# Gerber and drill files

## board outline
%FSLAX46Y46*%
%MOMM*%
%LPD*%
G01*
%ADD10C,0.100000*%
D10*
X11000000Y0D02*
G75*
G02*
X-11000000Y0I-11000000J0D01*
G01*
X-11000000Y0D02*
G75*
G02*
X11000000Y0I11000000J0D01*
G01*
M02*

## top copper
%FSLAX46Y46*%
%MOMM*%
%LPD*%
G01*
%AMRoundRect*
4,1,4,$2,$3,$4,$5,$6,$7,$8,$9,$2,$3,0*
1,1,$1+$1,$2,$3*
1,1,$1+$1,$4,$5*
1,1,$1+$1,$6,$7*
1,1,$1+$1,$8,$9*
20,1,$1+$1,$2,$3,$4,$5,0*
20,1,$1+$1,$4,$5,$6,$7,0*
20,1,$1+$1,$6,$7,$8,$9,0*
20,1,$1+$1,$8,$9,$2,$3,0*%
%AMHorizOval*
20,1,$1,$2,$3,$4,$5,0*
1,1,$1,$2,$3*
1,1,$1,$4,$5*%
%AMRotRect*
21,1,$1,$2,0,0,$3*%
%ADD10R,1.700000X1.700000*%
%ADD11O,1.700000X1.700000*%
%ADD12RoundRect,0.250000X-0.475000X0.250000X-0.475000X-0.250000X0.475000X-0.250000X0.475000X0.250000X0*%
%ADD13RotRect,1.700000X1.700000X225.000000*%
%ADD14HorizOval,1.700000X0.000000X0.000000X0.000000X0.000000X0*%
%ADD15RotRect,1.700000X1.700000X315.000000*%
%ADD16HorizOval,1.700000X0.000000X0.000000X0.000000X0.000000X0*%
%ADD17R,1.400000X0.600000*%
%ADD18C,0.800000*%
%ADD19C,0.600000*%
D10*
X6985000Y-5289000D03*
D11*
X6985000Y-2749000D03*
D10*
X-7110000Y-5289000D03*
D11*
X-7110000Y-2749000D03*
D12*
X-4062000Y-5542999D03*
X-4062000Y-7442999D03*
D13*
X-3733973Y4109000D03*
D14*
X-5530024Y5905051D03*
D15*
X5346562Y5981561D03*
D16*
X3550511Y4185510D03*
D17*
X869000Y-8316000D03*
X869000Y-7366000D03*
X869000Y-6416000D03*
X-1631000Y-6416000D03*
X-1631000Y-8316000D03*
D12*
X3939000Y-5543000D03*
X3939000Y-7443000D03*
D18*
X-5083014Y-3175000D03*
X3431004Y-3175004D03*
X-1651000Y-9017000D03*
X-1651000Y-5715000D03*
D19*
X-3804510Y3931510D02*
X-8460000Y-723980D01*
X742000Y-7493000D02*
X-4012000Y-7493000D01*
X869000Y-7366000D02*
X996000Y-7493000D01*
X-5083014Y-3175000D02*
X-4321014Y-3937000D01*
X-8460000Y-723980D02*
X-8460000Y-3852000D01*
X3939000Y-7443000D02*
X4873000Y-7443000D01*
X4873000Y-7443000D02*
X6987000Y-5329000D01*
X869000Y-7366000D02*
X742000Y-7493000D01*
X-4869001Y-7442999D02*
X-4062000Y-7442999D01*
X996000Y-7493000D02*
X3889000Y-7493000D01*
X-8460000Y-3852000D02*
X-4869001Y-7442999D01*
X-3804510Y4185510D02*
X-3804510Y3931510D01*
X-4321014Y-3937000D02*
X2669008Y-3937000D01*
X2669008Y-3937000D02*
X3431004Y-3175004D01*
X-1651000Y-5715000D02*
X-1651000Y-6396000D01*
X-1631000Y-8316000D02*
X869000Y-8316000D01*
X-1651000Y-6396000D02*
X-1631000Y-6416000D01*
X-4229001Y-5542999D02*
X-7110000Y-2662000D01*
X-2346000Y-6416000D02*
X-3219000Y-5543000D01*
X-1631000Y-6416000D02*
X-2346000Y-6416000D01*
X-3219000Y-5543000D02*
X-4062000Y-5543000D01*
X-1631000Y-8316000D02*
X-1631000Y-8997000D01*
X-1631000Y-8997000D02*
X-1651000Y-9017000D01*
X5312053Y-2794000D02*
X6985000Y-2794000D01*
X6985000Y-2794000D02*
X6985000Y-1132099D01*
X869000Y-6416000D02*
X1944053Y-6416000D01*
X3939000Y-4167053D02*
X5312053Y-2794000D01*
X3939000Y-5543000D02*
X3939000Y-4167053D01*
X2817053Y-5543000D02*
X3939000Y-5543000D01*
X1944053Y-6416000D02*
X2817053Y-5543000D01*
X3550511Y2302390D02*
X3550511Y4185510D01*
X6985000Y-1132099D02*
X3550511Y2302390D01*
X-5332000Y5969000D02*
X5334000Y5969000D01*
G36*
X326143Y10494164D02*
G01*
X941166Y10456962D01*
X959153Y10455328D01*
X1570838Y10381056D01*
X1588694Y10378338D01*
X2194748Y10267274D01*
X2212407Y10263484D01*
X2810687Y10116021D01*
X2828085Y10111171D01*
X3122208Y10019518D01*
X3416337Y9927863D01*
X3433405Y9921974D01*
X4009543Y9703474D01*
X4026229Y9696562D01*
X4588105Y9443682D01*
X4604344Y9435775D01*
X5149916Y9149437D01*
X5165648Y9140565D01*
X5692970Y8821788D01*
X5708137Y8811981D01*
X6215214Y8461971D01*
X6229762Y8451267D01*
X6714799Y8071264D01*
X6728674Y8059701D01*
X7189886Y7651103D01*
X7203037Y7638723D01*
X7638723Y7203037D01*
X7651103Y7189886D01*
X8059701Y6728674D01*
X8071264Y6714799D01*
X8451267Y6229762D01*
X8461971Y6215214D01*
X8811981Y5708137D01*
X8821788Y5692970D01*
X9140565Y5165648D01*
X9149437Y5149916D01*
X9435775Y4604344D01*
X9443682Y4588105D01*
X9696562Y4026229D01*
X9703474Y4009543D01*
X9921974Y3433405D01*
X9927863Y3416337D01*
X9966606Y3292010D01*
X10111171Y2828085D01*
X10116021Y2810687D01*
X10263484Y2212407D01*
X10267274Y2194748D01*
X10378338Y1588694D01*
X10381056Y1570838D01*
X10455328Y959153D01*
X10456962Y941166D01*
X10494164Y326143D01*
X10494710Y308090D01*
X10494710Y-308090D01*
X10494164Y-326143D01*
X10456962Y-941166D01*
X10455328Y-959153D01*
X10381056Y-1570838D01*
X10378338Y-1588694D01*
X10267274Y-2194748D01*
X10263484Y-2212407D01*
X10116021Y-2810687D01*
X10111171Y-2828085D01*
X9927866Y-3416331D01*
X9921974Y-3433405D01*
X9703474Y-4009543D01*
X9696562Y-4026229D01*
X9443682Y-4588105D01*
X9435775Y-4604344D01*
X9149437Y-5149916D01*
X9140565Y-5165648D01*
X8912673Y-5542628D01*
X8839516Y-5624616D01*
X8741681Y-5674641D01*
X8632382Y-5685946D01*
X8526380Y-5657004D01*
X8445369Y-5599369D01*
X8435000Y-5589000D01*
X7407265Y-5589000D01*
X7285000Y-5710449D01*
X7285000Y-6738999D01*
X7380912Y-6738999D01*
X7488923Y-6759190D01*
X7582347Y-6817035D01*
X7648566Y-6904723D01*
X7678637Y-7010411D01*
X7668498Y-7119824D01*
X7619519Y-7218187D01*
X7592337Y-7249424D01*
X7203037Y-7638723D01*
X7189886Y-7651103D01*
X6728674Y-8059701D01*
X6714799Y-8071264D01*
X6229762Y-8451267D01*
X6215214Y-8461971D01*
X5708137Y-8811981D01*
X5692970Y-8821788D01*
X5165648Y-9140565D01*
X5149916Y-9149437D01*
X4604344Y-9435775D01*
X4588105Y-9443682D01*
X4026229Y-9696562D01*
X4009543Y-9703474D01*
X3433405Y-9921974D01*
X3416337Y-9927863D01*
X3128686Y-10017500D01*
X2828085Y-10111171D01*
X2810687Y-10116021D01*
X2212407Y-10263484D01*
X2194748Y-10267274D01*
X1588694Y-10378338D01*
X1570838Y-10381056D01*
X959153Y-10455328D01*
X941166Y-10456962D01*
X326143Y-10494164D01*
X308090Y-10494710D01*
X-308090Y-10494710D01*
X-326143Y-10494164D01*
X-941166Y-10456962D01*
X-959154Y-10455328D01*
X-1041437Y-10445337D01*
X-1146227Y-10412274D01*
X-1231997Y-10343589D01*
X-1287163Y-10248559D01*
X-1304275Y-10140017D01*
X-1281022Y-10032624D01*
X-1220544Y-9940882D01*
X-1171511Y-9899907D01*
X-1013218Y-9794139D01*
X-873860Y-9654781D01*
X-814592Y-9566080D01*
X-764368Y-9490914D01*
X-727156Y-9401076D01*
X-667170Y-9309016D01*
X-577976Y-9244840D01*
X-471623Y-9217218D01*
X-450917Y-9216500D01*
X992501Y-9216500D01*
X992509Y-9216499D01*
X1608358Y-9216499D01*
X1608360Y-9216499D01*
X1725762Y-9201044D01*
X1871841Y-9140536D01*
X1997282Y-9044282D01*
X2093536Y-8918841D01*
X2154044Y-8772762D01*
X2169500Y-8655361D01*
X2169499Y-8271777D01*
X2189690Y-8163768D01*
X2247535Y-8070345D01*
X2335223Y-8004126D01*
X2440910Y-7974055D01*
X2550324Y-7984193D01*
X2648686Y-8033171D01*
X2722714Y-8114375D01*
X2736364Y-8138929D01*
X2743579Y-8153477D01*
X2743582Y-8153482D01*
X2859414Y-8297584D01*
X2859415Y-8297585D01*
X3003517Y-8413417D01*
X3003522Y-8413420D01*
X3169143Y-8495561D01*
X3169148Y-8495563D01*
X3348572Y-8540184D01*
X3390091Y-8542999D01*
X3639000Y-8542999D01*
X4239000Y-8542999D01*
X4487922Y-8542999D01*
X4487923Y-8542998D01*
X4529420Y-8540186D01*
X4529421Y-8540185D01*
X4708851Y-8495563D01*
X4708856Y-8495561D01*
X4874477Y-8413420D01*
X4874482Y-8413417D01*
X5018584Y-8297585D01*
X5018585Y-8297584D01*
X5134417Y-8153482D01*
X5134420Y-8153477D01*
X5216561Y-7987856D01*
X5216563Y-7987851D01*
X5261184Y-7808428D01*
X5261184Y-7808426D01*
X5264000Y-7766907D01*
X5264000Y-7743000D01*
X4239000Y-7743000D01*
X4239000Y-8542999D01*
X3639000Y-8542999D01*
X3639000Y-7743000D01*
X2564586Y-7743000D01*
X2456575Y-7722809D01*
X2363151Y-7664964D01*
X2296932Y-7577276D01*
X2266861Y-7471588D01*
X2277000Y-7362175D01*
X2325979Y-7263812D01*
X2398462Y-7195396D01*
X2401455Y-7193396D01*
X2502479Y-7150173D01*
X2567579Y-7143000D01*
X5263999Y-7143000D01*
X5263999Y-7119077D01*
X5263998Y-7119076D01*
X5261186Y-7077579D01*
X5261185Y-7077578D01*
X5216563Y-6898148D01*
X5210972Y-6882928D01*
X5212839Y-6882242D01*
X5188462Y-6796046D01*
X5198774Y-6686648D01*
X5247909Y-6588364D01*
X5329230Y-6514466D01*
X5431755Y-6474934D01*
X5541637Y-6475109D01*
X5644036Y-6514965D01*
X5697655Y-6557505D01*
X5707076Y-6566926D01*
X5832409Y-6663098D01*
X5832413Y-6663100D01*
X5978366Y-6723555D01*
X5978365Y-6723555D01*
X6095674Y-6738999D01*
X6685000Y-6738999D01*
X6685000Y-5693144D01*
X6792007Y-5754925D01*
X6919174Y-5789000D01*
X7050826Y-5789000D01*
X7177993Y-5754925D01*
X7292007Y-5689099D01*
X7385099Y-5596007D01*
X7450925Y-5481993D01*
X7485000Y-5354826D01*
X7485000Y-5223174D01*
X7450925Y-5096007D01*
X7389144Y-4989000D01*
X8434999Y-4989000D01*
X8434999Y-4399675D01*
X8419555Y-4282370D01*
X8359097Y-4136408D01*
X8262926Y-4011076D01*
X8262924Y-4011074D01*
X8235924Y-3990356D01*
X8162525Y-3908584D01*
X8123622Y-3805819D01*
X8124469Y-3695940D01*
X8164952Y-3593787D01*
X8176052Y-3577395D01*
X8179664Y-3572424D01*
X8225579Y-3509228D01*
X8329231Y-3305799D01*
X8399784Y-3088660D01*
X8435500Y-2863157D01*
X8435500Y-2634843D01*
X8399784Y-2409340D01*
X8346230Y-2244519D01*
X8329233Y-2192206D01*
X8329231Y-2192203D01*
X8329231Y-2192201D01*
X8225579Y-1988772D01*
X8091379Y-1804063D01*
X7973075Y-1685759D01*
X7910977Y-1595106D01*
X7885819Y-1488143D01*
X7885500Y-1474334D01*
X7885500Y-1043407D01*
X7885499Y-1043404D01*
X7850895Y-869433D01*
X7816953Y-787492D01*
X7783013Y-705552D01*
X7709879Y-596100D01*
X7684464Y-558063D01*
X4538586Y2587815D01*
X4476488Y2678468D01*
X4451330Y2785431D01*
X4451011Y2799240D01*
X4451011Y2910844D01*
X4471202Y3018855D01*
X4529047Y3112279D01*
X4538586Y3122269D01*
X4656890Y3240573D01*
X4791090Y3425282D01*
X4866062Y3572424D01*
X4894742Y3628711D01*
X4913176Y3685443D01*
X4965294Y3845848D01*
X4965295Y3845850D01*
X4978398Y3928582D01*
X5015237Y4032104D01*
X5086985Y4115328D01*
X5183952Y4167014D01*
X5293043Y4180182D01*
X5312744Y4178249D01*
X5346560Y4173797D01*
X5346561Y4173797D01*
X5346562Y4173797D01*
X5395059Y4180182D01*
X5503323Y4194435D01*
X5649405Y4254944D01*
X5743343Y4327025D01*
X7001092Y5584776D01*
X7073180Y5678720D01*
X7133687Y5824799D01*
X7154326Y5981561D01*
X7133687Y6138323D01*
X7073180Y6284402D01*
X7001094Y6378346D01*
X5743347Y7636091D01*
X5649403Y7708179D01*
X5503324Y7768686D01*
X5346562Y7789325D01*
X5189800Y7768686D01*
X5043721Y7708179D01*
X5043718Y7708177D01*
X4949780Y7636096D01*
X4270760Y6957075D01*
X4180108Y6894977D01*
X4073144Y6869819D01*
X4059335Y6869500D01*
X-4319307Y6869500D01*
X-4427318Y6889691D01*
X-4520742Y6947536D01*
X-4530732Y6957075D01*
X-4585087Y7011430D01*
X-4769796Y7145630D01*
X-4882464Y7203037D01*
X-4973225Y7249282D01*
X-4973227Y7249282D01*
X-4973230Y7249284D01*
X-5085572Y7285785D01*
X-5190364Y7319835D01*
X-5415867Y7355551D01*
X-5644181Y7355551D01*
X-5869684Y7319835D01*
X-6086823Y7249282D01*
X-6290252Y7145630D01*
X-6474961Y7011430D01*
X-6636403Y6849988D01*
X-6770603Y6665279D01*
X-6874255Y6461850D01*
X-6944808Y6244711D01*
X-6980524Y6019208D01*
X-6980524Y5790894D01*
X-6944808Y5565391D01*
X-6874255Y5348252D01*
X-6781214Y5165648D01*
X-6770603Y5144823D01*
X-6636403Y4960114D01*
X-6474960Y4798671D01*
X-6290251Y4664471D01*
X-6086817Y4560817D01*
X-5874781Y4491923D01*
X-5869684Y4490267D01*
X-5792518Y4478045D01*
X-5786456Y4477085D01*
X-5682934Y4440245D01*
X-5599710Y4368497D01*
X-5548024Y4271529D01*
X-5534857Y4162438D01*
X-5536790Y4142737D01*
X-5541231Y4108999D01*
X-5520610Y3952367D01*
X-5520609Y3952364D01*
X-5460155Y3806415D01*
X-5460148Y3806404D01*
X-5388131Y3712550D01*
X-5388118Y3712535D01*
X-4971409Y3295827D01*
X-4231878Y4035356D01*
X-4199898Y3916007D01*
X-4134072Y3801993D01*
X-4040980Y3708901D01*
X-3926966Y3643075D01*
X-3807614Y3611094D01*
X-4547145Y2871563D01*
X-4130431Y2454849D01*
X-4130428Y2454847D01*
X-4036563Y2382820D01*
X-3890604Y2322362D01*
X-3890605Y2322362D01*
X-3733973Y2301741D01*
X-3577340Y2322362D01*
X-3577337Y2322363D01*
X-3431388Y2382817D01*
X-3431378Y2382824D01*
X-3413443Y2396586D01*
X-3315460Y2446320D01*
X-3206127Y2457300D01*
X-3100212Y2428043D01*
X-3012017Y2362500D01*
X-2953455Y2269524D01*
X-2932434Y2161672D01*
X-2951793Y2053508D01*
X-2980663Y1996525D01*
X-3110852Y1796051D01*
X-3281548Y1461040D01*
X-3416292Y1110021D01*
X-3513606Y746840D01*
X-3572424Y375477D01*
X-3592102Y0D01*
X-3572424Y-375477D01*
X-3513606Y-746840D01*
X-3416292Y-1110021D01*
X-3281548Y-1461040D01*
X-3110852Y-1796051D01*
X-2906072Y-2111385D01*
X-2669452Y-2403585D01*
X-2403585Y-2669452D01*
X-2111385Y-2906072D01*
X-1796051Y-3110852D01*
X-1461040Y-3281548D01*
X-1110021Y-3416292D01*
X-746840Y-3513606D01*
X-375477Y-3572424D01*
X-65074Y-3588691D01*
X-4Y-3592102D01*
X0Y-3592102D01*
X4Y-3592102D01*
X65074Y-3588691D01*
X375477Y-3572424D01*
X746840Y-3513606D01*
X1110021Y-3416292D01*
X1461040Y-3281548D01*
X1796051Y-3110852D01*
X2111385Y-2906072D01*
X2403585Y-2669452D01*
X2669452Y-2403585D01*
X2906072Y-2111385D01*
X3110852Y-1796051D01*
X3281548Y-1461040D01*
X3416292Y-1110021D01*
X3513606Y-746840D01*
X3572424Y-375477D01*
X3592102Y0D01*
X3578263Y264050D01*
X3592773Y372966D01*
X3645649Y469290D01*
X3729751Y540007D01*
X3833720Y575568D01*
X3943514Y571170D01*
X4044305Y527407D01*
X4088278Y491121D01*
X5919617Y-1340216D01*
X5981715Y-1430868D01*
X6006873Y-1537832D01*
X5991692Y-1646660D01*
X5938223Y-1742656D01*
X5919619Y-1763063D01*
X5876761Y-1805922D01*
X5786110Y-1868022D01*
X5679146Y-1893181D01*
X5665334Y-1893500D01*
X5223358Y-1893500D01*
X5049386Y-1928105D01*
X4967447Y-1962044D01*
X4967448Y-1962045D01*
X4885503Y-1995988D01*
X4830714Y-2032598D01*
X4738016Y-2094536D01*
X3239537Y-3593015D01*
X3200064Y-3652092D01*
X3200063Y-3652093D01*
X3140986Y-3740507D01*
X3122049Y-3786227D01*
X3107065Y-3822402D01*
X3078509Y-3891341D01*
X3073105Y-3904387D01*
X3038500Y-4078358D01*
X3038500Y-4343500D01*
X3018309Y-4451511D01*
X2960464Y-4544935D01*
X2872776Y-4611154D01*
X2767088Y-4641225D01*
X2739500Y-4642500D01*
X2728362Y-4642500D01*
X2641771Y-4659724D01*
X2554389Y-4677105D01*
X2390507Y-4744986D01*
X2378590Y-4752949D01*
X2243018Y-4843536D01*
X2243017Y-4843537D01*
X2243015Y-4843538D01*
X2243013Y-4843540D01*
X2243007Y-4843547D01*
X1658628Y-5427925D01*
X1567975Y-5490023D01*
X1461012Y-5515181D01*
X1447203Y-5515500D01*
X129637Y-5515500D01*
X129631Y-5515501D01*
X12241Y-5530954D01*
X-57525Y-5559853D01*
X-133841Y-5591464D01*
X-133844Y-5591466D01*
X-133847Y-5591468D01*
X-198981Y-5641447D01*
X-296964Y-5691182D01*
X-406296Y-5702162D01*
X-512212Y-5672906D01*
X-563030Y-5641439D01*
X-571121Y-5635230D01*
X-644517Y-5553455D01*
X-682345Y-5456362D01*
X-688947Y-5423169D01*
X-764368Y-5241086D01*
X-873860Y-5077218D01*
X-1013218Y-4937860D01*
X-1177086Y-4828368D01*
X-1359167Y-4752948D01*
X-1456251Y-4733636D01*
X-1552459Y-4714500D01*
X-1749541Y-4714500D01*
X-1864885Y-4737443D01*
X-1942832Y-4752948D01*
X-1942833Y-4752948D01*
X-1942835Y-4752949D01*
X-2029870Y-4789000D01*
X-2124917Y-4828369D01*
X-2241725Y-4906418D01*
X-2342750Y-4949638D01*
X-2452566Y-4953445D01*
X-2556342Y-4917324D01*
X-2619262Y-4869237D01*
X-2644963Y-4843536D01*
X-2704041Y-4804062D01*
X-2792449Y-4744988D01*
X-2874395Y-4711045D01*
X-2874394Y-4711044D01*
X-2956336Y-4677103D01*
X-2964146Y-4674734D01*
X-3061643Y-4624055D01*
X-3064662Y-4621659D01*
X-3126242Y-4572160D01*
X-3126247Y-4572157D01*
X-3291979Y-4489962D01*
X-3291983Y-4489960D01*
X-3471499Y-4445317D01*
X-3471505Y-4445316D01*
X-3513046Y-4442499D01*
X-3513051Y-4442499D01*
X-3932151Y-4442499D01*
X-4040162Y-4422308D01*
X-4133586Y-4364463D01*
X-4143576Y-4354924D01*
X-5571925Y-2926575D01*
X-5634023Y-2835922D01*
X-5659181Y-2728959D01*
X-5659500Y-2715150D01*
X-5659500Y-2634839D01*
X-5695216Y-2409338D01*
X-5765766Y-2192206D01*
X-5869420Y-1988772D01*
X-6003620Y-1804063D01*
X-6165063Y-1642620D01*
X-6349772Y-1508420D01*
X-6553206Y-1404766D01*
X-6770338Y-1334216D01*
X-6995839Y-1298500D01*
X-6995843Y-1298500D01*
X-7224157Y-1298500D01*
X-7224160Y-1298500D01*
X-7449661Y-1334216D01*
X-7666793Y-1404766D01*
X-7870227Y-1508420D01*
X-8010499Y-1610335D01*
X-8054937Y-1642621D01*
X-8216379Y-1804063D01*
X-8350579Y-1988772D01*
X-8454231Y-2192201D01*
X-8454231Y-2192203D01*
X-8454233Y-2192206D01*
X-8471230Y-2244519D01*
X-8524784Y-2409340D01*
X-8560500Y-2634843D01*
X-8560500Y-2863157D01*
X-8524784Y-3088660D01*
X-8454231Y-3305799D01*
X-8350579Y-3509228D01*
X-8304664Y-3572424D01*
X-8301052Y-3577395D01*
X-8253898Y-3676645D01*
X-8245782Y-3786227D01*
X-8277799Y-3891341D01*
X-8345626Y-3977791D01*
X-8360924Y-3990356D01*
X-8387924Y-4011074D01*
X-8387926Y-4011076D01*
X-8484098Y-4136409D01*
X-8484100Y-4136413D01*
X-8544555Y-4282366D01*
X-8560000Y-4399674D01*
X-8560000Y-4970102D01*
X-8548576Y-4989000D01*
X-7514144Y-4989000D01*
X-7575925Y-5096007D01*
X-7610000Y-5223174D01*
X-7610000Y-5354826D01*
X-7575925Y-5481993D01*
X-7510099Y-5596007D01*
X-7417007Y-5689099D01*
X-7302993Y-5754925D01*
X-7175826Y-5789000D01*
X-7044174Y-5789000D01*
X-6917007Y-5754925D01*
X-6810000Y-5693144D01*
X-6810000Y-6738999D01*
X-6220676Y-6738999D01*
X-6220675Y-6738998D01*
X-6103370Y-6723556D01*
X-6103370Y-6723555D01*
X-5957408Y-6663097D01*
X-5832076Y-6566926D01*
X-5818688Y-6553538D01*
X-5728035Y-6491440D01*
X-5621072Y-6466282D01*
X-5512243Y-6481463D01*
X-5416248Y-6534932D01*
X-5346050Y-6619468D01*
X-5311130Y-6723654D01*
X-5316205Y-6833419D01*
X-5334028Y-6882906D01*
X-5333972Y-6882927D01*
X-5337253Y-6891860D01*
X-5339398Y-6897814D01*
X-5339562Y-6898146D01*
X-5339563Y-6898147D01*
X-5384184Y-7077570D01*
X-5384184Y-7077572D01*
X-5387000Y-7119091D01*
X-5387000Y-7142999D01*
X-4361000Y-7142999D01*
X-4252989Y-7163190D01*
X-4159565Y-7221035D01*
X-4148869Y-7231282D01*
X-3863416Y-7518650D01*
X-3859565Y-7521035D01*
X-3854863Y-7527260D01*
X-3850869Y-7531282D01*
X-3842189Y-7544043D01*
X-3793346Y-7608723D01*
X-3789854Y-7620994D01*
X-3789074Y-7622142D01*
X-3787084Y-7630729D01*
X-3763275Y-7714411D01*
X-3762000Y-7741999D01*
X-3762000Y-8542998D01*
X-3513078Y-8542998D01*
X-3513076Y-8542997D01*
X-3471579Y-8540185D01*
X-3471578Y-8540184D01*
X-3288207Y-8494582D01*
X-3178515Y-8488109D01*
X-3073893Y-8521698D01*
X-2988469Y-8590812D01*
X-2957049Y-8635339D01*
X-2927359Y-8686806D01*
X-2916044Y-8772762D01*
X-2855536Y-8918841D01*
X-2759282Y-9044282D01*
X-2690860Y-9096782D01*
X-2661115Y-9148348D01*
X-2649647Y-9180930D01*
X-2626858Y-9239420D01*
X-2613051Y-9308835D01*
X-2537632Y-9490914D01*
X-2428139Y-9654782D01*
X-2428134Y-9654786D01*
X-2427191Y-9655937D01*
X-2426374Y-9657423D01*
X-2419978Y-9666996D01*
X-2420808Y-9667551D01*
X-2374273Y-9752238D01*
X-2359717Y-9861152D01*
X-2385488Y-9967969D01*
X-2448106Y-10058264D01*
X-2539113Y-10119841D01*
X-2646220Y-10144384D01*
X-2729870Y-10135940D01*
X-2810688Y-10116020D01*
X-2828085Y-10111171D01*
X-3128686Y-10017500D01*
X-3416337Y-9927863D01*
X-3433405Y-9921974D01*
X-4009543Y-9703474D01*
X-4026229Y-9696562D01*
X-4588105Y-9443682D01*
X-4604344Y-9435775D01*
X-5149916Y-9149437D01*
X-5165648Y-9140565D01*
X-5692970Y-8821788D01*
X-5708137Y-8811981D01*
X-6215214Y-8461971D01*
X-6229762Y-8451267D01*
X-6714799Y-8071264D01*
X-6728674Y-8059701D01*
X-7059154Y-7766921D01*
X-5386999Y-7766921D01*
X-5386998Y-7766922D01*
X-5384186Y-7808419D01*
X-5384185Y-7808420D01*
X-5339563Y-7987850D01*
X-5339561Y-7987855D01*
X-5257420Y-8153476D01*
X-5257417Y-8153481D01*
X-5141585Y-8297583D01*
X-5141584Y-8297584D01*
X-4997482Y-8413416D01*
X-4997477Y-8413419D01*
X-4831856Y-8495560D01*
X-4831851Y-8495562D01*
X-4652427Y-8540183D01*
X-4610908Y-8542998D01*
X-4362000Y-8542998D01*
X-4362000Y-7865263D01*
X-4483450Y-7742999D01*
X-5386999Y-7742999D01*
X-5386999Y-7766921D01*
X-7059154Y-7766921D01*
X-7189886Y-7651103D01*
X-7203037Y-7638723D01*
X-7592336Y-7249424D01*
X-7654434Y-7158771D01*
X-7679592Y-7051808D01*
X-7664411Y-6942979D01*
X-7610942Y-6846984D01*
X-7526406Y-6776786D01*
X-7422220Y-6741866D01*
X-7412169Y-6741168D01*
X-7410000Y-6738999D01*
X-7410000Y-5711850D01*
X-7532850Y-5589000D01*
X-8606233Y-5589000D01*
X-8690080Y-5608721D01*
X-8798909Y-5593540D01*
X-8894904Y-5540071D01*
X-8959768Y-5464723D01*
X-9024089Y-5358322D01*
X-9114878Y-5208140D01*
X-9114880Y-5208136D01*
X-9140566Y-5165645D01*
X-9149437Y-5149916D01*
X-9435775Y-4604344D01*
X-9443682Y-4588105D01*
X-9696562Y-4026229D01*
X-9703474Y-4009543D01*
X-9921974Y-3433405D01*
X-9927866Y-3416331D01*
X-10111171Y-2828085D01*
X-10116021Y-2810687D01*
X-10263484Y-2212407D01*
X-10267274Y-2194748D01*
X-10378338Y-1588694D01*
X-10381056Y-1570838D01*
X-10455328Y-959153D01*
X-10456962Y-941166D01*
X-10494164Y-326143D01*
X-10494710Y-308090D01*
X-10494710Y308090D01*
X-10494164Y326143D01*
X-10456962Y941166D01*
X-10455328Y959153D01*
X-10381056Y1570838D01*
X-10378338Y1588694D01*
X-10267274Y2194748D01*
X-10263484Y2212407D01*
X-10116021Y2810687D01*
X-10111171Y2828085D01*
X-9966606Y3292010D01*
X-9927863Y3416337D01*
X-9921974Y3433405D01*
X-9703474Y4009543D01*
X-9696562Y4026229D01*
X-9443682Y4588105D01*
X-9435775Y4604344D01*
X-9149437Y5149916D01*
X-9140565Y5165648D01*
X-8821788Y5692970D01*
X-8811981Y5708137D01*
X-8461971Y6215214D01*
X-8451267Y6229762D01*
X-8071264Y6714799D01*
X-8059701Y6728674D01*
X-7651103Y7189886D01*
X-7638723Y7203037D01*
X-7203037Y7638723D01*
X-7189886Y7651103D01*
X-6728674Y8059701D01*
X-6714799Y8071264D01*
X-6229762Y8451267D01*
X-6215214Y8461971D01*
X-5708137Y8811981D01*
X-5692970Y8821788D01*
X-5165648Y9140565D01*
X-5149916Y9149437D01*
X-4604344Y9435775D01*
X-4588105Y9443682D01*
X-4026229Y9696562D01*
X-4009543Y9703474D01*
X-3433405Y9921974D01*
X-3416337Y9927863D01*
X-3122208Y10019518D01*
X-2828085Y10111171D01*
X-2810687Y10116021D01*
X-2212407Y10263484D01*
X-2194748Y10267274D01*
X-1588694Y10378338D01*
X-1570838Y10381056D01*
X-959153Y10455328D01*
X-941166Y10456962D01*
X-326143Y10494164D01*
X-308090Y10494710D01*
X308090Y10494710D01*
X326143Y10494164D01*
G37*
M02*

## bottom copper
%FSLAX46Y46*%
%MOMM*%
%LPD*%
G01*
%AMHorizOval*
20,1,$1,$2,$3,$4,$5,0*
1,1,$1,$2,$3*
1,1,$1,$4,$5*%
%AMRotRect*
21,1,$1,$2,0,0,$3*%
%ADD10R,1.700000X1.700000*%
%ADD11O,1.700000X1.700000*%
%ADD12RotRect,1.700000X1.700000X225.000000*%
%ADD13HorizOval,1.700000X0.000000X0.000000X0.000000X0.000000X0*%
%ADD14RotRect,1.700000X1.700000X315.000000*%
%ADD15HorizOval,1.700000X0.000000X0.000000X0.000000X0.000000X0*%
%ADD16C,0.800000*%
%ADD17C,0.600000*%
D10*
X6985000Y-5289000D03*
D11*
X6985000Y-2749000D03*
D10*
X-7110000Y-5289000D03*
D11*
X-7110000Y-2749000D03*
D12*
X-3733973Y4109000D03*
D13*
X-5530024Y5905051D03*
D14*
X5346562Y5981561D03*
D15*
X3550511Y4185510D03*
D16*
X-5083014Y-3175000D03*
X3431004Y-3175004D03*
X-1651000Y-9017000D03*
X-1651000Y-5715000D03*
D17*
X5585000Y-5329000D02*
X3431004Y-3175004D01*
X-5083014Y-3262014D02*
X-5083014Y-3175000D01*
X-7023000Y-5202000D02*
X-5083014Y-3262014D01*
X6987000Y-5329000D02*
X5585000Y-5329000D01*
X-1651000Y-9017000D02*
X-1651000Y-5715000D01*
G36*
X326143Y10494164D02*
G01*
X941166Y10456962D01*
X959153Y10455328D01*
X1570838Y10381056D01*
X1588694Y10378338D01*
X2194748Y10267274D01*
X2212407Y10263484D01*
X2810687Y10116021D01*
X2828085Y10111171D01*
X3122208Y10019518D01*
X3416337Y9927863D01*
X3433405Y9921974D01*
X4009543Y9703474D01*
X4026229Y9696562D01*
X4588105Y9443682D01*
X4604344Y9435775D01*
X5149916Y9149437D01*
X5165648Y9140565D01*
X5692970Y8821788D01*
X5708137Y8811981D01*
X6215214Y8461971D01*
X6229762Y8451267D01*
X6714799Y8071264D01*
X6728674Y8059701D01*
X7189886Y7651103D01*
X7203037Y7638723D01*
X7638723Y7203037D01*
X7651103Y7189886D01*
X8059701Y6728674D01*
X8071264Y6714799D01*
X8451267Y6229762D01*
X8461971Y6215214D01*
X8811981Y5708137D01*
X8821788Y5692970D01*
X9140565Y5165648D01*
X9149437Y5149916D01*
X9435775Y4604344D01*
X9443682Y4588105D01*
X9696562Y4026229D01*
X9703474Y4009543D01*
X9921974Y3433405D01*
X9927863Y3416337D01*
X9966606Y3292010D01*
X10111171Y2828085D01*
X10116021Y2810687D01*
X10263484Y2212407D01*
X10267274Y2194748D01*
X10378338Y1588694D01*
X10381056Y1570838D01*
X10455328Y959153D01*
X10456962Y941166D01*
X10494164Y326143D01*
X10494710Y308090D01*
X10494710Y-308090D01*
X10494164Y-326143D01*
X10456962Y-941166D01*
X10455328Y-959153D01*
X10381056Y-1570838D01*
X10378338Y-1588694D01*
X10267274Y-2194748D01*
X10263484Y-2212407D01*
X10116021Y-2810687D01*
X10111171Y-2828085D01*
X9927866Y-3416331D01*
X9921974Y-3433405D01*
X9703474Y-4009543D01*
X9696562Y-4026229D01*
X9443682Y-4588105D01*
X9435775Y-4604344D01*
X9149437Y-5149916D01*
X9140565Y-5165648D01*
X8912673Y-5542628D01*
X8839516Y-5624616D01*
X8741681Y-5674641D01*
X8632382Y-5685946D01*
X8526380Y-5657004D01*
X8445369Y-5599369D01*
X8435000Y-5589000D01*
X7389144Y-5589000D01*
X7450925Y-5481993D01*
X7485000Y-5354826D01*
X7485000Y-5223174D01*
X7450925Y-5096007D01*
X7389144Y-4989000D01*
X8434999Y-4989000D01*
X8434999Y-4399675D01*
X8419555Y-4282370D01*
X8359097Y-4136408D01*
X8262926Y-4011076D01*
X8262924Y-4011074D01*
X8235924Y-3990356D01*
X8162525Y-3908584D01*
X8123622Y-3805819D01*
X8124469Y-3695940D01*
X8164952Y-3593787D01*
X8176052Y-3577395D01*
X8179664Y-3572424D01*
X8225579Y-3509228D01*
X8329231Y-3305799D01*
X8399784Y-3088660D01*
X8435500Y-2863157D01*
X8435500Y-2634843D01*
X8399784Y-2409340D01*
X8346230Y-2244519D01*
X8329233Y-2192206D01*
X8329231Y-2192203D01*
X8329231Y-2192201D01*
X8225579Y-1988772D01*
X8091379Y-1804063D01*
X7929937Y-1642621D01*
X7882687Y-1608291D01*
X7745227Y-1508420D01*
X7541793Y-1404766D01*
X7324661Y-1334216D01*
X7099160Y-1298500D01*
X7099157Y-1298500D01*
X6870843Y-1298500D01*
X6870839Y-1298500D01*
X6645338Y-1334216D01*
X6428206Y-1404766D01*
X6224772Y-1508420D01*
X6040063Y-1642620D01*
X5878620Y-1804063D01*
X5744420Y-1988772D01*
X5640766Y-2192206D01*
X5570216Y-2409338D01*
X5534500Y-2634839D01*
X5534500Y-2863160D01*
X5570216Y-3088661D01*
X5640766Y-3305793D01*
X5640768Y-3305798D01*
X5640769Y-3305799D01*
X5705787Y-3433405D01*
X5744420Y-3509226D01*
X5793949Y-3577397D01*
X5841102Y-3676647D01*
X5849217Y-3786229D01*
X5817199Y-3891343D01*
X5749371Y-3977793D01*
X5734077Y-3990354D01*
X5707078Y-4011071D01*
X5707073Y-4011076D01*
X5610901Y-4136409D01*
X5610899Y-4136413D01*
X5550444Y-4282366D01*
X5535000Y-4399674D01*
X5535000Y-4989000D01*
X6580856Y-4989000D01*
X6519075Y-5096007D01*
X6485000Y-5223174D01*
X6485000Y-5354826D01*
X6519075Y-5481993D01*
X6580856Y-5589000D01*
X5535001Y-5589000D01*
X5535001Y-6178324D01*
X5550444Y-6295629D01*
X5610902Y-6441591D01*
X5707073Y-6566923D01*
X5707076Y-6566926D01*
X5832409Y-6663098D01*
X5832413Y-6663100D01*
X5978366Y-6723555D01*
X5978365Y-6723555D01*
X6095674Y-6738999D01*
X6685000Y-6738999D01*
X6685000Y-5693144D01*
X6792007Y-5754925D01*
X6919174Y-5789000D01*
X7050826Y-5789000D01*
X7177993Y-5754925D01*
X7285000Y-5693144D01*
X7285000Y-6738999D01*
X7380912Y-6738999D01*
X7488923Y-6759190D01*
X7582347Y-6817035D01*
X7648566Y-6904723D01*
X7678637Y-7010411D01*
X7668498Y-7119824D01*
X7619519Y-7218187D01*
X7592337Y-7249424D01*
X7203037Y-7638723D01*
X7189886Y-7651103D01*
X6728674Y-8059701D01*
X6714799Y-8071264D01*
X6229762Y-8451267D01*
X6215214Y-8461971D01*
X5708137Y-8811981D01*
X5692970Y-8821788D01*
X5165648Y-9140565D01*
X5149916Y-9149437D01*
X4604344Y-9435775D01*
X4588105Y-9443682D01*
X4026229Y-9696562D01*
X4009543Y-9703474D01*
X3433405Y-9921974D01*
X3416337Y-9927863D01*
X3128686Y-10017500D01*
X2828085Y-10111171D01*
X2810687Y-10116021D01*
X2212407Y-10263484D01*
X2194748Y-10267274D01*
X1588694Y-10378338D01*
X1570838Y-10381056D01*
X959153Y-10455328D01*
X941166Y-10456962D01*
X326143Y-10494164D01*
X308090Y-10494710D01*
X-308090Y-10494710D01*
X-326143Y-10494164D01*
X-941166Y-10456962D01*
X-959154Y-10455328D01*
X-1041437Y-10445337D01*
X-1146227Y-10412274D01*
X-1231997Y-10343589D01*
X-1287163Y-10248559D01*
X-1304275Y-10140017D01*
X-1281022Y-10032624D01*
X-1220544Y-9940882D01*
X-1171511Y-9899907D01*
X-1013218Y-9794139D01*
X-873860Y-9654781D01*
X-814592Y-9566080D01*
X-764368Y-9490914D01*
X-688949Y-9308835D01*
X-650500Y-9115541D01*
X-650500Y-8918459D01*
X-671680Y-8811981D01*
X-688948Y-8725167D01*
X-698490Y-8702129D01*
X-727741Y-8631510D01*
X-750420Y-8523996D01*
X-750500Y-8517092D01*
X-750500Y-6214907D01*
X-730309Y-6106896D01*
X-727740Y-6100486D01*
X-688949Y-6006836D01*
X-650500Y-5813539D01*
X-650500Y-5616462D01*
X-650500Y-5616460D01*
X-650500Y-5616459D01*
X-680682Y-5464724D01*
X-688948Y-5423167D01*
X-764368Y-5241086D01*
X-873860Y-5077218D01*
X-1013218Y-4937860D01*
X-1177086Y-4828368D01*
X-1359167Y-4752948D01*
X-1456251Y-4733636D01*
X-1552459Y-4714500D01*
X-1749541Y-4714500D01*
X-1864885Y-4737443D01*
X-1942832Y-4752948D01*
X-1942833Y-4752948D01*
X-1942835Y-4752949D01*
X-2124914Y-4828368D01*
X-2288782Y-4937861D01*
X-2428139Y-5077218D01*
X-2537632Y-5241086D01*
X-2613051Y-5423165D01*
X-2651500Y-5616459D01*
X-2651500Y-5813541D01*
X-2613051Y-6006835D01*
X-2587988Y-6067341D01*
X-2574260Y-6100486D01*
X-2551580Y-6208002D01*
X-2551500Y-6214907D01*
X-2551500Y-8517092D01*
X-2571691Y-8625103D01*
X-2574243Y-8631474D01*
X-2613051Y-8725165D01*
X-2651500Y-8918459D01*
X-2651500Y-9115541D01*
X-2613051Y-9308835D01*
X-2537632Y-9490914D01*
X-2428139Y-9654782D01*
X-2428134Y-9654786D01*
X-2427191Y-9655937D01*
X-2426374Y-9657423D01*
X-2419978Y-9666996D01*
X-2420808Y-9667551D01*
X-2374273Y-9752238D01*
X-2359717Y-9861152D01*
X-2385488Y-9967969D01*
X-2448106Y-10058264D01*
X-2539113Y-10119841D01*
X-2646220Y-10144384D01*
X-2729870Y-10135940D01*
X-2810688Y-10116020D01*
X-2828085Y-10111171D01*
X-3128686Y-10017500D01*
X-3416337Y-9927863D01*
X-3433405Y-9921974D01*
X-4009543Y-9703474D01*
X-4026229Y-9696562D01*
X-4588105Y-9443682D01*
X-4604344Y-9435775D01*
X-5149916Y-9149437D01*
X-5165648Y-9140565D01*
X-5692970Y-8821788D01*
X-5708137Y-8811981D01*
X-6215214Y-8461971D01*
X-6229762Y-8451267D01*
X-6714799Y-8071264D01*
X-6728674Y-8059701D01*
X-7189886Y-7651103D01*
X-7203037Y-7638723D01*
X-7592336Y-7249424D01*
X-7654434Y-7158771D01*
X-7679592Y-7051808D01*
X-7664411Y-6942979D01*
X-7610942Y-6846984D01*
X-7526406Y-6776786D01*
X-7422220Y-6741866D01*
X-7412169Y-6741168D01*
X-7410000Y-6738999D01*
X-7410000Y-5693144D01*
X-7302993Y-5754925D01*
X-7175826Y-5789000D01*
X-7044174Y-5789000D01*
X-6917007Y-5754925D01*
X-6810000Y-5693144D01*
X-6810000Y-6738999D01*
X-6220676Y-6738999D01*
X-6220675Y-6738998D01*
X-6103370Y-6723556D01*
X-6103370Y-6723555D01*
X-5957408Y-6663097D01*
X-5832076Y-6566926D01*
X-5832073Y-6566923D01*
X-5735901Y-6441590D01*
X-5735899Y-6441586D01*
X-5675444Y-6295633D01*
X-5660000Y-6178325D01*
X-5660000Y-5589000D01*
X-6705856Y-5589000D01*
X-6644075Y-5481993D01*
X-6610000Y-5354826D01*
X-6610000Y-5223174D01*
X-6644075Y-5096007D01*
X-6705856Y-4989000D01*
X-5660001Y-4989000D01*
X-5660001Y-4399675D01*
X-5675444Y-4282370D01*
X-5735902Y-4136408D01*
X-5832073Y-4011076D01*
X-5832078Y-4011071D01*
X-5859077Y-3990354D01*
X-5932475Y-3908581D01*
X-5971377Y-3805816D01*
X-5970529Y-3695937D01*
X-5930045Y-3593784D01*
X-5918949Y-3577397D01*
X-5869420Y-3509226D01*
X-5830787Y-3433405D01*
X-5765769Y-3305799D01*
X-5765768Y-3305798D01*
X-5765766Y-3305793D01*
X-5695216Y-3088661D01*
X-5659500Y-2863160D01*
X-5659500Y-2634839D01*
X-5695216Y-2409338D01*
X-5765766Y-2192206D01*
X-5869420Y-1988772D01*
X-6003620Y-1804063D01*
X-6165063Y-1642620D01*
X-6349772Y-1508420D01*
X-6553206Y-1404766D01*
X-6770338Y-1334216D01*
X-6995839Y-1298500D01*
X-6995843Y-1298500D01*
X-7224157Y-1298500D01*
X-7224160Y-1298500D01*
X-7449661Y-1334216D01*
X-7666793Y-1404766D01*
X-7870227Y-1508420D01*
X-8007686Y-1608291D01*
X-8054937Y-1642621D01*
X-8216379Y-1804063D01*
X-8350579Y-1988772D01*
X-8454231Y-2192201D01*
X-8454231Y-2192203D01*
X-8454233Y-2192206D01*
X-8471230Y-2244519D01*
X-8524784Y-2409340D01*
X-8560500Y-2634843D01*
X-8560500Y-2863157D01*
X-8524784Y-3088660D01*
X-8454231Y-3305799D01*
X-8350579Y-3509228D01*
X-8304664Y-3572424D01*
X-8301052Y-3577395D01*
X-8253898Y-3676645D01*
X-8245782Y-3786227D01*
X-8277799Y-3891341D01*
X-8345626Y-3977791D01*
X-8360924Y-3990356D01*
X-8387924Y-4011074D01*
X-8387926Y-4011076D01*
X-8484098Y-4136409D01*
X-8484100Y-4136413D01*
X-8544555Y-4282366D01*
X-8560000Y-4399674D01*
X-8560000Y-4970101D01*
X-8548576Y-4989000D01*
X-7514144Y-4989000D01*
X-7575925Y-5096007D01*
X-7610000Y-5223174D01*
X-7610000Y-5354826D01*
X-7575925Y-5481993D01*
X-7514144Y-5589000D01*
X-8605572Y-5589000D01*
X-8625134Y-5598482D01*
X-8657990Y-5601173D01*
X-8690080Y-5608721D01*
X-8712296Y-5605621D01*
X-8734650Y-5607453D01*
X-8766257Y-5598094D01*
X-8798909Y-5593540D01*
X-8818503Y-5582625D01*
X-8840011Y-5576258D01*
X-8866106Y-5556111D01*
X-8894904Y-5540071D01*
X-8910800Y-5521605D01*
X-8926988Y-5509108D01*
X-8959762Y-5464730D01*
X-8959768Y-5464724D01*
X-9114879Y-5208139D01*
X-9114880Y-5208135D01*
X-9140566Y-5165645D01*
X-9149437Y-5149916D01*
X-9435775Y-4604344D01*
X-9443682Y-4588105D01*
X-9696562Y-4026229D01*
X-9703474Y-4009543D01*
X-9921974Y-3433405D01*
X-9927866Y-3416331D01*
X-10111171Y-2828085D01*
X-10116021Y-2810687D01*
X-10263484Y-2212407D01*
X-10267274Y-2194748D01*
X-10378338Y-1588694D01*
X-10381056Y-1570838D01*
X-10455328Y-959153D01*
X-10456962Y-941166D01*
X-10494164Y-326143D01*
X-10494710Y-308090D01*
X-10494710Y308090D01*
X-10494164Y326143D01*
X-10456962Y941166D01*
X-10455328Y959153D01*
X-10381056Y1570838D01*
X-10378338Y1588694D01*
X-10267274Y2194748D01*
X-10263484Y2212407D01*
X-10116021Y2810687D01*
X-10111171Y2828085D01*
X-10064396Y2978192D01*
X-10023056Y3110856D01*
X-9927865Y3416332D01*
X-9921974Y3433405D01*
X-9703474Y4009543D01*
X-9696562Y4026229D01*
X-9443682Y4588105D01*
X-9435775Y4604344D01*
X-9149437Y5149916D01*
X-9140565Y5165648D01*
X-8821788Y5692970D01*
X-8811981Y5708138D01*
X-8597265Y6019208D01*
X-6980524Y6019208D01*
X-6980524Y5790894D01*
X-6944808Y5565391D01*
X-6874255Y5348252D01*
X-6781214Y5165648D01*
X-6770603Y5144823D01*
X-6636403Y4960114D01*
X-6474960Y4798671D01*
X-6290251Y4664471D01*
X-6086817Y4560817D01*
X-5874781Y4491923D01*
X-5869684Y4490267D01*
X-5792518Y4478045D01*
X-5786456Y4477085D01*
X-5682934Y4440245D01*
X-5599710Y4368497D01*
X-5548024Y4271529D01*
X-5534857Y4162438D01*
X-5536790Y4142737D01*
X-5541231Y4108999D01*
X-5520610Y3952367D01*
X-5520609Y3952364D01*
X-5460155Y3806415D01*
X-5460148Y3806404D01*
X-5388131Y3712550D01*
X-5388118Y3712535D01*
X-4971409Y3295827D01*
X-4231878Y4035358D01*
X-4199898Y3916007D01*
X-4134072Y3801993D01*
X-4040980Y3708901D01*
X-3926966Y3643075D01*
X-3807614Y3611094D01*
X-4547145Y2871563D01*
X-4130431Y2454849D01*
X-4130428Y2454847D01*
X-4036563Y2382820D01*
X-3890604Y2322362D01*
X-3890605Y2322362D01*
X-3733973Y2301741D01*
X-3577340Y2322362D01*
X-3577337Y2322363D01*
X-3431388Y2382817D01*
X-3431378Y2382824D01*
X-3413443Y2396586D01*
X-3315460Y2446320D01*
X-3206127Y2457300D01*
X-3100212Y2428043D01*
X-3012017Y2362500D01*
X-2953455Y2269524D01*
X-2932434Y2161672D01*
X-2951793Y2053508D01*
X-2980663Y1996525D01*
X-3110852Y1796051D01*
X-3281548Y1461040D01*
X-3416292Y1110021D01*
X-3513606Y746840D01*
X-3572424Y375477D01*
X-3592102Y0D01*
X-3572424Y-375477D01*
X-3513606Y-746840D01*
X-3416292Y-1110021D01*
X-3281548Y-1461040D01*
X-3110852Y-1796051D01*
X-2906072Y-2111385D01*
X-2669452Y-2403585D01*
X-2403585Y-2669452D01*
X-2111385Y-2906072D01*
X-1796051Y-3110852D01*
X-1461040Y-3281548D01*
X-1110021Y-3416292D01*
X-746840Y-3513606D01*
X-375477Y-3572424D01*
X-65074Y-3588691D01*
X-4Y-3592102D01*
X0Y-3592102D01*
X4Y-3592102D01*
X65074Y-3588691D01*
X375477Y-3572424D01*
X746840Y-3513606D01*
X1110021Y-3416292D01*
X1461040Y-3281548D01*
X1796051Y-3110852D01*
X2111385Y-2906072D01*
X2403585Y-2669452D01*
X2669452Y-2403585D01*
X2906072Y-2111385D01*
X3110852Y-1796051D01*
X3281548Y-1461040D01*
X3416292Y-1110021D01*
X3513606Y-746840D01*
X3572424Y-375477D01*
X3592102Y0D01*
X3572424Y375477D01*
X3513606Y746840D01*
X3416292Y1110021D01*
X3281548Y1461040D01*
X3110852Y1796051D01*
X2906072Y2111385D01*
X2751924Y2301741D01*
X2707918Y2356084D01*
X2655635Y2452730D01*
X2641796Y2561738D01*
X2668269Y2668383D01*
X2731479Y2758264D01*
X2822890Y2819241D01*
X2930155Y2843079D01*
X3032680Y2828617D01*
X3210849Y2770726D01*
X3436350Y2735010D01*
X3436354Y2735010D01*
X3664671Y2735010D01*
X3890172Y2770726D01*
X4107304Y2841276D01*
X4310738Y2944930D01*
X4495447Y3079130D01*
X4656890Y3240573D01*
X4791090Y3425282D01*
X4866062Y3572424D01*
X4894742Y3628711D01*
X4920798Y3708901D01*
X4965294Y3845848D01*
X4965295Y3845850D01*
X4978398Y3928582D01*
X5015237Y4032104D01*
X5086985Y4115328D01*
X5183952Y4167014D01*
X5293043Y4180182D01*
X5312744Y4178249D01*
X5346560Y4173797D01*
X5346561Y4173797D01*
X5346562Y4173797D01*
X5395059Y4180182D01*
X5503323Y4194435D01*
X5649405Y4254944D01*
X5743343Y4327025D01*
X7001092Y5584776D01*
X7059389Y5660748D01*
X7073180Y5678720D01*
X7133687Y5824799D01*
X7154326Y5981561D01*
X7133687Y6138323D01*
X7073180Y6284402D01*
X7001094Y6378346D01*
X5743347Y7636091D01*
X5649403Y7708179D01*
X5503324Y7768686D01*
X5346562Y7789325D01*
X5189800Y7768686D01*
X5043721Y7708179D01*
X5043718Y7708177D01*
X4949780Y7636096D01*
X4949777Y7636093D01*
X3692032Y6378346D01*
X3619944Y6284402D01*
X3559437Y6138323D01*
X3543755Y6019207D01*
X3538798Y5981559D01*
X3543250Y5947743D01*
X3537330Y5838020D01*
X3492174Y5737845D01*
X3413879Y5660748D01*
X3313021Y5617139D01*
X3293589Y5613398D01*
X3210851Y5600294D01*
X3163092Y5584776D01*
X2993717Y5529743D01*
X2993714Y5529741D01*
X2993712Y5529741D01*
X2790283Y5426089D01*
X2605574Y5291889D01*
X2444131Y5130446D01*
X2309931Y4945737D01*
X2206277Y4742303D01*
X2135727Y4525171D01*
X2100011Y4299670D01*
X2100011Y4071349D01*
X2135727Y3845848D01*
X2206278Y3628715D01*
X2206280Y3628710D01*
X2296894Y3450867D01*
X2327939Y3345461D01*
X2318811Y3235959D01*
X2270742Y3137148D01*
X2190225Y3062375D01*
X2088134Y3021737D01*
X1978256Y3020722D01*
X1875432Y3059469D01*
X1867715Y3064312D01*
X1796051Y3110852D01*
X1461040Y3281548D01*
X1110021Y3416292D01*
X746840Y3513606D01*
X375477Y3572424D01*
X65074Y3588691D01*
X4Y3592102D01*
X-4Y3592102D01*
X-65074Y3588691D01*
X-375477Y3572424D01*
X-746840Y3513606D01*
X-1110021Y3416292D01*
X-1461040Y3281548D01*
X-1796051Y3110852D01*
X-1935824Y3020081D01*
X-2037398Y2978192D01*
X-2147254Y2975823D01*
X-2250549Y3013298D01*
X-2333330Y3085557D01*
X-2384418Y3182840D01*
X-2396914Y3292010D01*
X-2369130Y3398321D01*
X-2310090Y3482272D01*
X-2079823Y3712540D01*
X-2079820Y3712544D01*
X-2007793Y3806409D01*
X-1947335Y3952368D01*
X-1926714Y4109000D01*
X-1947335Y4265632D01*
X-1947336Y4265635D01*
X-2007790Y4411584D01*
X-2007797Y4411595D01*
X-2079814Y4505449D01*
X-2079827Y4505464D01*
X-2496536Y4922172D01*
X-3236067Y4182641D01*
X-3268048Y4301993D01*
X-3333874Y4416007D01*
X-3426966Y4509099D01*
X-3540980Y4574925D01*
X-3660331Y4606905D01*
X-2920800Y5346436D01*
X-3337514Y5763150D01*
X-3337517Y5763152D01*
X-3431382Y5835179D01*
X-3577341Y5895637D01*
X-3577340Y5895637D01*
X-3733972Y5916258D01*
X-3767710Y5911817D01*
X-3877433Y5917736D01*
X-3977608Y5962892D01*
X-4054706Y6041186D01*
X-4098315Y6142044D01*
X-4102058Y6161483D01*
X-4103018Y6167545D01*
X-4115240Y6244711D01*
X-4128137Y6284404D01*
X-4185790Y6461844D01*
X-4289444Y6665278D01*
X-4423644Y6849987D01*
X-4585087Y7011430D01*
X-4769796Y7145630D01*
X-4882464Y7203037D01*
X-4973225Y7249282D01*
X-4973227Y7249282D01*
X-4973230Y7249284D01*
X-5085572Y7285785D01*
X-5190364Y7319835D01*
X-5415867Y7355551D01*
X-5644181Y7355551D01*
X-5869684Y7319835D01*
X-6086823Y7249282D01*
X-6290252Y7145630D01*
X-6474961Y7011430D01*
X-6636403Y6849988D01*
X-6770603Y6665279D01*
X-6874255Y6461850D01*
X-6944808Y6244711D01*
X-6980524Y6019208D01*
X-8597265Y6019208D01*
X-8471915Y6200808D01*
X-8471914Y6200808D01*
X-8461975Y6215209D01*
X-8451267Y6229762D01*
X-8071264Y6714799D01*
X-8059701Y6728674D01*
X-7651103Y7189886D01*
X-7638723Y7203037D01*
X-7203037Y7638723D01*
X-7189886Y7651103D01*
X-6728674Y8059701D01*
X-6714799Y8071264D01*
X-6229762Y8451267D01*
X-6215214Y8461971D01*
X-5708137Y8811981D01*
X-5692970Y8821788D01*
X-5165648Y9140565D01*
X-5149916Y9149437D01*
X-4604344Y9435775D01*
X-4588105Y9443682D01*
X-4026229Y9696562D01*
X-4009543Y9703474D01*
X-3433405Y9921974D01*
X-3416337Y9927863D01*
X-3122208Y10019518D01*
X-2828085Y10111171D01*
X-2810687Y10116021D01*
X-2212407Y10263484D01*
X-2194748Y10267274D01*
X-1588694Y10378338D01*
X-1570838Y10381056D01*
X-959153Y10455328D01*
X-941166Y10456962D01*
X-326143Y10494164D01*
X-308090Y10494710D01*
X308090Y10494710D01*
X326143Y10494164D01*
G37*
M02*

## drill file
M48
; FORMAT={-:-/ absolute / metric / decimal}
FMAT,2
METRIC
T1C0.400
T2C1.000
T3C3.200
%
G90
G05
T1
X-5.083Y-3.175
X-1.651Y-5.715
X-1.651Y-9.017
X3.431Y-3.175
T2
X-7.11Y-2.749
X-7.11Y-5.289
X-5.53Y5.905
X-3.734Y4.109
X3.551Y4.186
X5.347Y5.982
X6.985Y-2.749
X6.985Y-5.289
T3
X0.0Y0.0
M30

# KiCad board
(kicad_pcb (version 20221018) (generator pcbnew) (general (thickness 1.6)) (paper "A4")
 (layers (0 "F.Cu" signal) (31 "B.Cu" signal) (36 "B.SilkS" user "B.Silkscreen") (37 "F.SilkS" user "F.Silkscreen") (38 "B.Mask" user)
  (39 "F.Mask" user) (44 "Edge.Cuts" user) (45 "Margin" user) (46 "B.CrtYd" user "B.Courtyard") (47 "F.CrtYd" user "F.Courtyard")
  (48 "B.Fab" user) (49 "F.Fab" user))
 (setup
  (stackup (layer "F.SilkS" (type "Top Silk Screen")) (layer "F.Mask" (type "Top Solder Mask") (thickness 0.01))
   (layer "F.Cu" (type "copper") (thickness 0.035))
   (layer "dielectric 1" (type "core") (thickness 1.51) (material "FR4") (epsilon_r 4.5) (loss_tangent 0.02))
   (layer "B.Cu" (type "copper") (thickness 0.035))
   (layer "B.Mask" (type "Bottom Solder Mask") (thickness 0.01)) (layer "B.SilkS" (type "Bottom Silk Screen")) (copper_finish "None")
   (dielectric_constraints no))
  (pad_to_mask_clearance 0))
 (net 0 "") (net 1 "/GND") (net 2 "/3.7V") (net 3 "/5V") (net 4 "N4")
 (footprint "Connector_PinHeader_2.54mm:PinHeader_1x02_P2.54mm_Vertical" (layer "F.Cu") (at 6.985 5.289 180)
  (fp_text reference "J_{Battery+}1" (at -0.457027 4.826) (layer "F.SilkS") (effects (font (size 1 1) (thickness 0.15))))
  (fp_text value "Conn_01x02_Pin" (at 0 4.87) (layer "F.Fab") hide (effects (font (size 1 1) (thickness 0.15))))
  (pad "1" thru_hole rect (at 0 0 180) (size 1.7 1.7) (drill 1) (layers "*.Cu" "*.Mask") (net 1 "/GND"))
  (pad "2" thru_hole oval (at 0 2.54 180) (size 1.7 1.7) (drill 1) (layers "*.Cu" "*.Mask") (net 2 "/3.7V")))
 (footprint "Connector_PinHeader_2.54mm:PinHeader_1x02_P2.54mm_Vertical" (layer "F.Cu") (at -7.11 5.289 180)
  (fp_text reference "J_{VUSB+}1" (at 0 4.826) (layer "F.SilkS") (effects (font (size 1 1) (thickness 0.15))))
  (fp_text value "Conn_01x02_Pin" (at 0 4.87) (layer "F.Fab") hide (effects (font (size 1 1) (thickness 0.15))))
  (pad "1" thru_hole rect (at 0 0 180) (size 1.7 1.7) (drill 1) (layers "*.Cu" "*.Mask") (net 1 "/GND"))
  (pad "2" thru_hole oval (at 0 2.54 180) (size 1.7 1.7) (drill 1) (layers "*.Cu" "*.Mask") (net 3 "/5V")))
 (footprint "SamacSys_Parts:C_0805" (layer "F.Cu") (at -4.062 6.476999 180)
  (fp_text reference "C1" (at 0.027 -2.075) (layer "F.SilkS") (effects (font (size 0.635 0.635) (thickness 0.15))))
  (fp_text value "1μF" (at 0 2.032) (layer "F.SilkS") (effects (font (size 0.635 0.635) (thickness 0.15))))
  (pad "1" smd roundrect (at 0 0.934 270) (size 1 1.45) (layers "F.Cu" "F.Paste" "F.Mask") (roundrect_rratio 0.25) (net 3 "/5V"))
  (pad "2" smd roundrect (at 0 -0.966 270) (size 1 1.45) (layers "F.Cu" "F.Paste" "F.Mask") (roundrect_rratio 0.25) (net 1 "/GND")))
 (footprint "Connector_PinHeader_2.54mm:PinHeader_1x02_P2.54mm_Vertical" (layer "F.Cu") (at -3.733973 -4.109 -135)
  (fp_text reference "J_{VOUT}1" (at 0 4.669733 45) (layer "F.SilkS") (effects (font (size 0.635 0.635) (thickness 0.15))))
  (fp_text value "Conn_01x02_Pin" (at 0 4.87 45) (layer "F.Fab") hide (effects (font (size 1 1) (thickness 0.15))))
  (pad "1" thru_hole rect (at 0 0 225) (size 1.7 1.7) (drill 1) (layers "*.Cu" "*.Mask") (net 1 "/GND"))
  (pad "2" thru_hole oval (at 0 2.54 225) (size 1.7 1.7) (drill 1) (layers "*.Cu" "*.Mask") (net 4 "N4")))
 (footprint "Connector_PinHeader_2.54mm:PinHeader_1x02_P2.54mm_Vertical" (layer "F.Cu") (at 5.346562 -5.981561 -45)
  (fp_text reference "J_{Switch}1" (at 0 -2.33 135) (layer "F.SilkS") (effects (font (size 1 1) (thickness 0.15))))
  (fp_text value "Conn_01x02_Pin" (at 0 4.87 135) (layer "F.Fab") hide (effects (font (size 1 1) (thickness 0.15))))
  (pad "1" thru_hole rect (at 0 0 315) (size 1.7 1.7) (drill 1) (layers "*.Cu" "*.Mask") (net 4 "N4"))
  (pad "2" thru_hole oval (at 0 2.54 315) (size 1.7 1.7) (drill 1) (layers "*.Cu" "*.Mask") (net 2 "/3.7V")))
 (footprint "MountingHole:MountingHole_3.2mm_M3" (layer "F.Cu") (at 0 0)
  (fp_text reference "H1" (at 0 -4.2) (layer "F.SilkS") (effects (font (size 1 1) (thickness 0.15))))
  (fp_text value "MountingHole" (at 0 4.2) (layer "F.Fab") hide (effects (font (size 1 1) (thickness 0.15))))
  (pad "" np_thru_hole circle (at 0 0) (size 3.2 3.2) (drill 3.2) (layers "*.Cu" "*.Mask")))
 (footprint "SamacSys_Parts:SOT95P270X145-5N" (layer "F.Cu") (at -0.381 7.366 180)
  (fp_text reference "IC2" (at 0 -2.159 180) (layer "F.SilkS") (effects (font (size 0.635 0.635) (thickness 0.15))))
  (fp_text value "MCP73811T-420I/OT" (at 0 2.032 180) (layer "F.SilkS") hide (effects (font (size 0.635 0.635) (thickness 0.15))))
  (pad "1" smd rect (at -1.25 -0.95 270) (size 0.6 1.4) (layers "F.Cu" "F.Paste" "F.Mask") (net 3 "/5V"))
  (pad "2" smd rect (at -1.25 0 270) (size 0.6 1.4) (layers "F.Cu" "F.Paste" "F.Mask") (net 1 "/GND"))
  (pad "3" smd rect (at -1.25 0.95 270) (size 0.6 1.4) (layers "F.Cu" "F.Paste" "F.Mask") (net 2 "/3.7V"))
  (pad "4" smd rect (at 1.25 0.95 270) (size 0.6 1.4) (layers "F.Cu" "F.Paste" "F.Mask") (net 3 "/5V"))
  (pad "5" smd rect (at 1.25 -0.95 270) (size 0.6 1.4) (layers "F.Cu" "F.Paste" "F.Mask") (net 3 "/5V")))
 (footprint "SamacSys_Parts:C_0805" (layer "F.Cu") (at 3.939 6.477 180)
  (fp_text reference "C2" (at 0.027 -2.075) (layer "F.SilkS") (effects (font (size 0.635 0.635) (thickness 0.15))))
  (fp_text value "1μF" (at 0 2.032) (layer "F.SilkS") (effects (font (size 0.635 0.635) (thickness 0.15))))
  (pad "1" smd roundrect (at 0 0.934 270) (size 1 1.45) (layers "F.Cu" "F.Paste" "F.Mask") (roundrect_rratio 0.25) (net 2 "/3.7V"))
  (pad "2" smd roundrect (at 0 -0.966 270) (size 1 1.45) (layers "F.Cu" "F.Paste" "F.Mask") (roundrect_rratio 0.25) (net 1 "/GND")))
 (gr_circle (center 0 0) (end 11 0) (stroke (width 0.1) (type default)) (fill none) (layer "Edge.Cuts"))
 (segment (start -3.80451 -3.93151) (end -8.46 0.72398) (width 0.6) (layer "F.Cu") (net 1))
 (segment (start 0.742 7.493) (end -4.012 7.493) (width 0.6) (layer "F.Cu") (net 1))
 (segment (start 0.869 7.366) (end 0.996 7.493) (width 0.6) (layer "F.Cu") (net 1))
 (segment (start -5.083014 3.175) (end -4.321014 3.937) (width 0.6) (layer "F.Cu") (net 1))
 (segment (start -8.46 0.72398) (end -8.46 3.852) (width 0.6) (layer "F.Cu") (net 1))
 (segment (start 3.939 7.443) (end 4.873 7.443) (width 0.6) (layer "F.Cu") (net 1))
 (segment (start 4.873 7.443) (end 6.987 5.329) (width 0.6) (layer "F.Cu") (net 1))
 (segment (start 0.869 7.366) (end 0.742 7.493) (width 0.6) (layer "F.Cu") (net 1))
 (segment (start -4.869001 7.442999) (end -4.062 7.442999) (width 0.6) (layer "F.Cu") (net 1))
 (segment (start 0.996 7.493) (end 3.889 7.493) (width 0.6) (layer "F.Cu") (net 1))
 (segment (start -8.46 3.852) (end -4.869001 7.442999) (width 0.6) (layer "F.Cu") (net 1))
 (segment (start -3.80451 -4.18551) (end -3.80451 -3.93151) (width 0.6) (layer "F.Cu") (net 1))
 (segment (start -4.321014 3.937) (end 2.669008 3.937) (width 0.6) (layer "F.Cu") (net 1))
 (segment (start 2.669008 3.937) (end 3.431004 3.175004) (width 0.6) (layer "F.Cu") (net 1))
 (via (at -5.083014 3.175) (size 0.8) (drill 0.4) (layers "F.Cu" "B.Cu") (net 1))
 (via (at 3.431004 3.175004) (size 0.8) (drill 0.4) (layers "F.Cu" "B.Cu") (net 1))
 (segment (start 5.585 5.329) (end 3.431004 3.175004) (width 0.6) (layer "B.Cu") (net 1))
 (segment (start -5.083014 3.262014) (end -5.083014 3.175) (width 0.6) (layer "B.Cu") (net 1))
 (segment (start -7.023 5.202) (end -5.083014 3.262014) (width 0.6) (layer "B.Cu") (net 1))
 (segment (start 6.987 5.329) (end 5.585 5.329) (width 0.6) (layer "B.Cu") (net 1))
 (segment (start -1.651 5.715) (end -1.651 6.396) (width 0.6) (layer "F.Cu") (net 3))
 (segment (start -1.631 8.316) (end 0.869 8.316) (width 0.6) (layer "F.Cu") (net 3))
 (segment (start -1.651 6.396) (end -1.631 6.416) (width 0.6) (layer "F.Cu") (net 3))
 (segment (start -4.229001 5.542999) (end -7.11 2.662) (width 0.6) (layer "F.Cu") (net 3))
 (segment (start -2.346 6.416) (end -3.219 5.543) (width 0.6) (layer "F.Cu") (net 3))
 (segment (start -1.631 6.416) (end -2.346 6.416) (width 0.6) (layer "F.Cu") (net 3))
 (segment (start -3.219 5.543) (end -4.062 5.543) (width 0.6) (layer "F.Cu") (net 3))
 (segment (start -1.631 8.316) (end -1.631 8.997) (width 0.6) (layer "F.Cu") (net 3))
 (segment (start -1.631 8.997) (end -1.651 9.017) (width 0.6) (layer "F.Cu") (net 3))
 (via (at -1.651 9.017) (size 0.8) (drill 0.4) (layers "F.Cu" "B.Cu") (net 3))
 (via (at -1.651 5.715) (size 0.8) (drill 0.4) (layers "F.Cu" "B.Cu") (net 3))
 (segment (start -1.651 9.017) (end -1.651 5.715) (width 0.6) (layer "B.Cu") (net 3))
 (segment (start 5.312053 2.794) (end 6.985 2.794) (width 0.6) (layer "F.Cu") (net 2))
 (segment (start 6.985 2.794) (end 6.985 1.132099) (width 0.6) (layer "F.Cu") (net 2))
 (segment (start 0.869 6.416) (end 1.944053 6.416) (width 0.6) (layer "F.Cu") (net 2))
 (segment (start 3.939 4.167053) (end 5.312053 2.794) (width 0.6) (layer "F.Cu") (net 2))
 (segment (start 3.939 5.543) (end 3.939 4.167053) (width 0.6) (layer "F.Cu") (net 2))
 (segment (start 2.817053 5.543) (end 3.939 5.543) (width 0.6) (layer "F.Cu") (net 2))
 (segment (start 1.944053 6.416) (end 2.817053 5.543) (width 0.6) (layer "F.Cu") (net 2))
 (segment (start 3.550511 -2.30239) (end 3.550511 -4.18551) (width 0.6) (layer "F.Cu") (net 2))
 (segment (start 6.985 1.132099) (end 3.550511 -2.30239) (width 0.6) (layer "F.Cu") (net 2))
 (segment (start -5.332 -5.969) (end 5.334 -5.969) (width 0.6) (layer "F.Cu") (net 4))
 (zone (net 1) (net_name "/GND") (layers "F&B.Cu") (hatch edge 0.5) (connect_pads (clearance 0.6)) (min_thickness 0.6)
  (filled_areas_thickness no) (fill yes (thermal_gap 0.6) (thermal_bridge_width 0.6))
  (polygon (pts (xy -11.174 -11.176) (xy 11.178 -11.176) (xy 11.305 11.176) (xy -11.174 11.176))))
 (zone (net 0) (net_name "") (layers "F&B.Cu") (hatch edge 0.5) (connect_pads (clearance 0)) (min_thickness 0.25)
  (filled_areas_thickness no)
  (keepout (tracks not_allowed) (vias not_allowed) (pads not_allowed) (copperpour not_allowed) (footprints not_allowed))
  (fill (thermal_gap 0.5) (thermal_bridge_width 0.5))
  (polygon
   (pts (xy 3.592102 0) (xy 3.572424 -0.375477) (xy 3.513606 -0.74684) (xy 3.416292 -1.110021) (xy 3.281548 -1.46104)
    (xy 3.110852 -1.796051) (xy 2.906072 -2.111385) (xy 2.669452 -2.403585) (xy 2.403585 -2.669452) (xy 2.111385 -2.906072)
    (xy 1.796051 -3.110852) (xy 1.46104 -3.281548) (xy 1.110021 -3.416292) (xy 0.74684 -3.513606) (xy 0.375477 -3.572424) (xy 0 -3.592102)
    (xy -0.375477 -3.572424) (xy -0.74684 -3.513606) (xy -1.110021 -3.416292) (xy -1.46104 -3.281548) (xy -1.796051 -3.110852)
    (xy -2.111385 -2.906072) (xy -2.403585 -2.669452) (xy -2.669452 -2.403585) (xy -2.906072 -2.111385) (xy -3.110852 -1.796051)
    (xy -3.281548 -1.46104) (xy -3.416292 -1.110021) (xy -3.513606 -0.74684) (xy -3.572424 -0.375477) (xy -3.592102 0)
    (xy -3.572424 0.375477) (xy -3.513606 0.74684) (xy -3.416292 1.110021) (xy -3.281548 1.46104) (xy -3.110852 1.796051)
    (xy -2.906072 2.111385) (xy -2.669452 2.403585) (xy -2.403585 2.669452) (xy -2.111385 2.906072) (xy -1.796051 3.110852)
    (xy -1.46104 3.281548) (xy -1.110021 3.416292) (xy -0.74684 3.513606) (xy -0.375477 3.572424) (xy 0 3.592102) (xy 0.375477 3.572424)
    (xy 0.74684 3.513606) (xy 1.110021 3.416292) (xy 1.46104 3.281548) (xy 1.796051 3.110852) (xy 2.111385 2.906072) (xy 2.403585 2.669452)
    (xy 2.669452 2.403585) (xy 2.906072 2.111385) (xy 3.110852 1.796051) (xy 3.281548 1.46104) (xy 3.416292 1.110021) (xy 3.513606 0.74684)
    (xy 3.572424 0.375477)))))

